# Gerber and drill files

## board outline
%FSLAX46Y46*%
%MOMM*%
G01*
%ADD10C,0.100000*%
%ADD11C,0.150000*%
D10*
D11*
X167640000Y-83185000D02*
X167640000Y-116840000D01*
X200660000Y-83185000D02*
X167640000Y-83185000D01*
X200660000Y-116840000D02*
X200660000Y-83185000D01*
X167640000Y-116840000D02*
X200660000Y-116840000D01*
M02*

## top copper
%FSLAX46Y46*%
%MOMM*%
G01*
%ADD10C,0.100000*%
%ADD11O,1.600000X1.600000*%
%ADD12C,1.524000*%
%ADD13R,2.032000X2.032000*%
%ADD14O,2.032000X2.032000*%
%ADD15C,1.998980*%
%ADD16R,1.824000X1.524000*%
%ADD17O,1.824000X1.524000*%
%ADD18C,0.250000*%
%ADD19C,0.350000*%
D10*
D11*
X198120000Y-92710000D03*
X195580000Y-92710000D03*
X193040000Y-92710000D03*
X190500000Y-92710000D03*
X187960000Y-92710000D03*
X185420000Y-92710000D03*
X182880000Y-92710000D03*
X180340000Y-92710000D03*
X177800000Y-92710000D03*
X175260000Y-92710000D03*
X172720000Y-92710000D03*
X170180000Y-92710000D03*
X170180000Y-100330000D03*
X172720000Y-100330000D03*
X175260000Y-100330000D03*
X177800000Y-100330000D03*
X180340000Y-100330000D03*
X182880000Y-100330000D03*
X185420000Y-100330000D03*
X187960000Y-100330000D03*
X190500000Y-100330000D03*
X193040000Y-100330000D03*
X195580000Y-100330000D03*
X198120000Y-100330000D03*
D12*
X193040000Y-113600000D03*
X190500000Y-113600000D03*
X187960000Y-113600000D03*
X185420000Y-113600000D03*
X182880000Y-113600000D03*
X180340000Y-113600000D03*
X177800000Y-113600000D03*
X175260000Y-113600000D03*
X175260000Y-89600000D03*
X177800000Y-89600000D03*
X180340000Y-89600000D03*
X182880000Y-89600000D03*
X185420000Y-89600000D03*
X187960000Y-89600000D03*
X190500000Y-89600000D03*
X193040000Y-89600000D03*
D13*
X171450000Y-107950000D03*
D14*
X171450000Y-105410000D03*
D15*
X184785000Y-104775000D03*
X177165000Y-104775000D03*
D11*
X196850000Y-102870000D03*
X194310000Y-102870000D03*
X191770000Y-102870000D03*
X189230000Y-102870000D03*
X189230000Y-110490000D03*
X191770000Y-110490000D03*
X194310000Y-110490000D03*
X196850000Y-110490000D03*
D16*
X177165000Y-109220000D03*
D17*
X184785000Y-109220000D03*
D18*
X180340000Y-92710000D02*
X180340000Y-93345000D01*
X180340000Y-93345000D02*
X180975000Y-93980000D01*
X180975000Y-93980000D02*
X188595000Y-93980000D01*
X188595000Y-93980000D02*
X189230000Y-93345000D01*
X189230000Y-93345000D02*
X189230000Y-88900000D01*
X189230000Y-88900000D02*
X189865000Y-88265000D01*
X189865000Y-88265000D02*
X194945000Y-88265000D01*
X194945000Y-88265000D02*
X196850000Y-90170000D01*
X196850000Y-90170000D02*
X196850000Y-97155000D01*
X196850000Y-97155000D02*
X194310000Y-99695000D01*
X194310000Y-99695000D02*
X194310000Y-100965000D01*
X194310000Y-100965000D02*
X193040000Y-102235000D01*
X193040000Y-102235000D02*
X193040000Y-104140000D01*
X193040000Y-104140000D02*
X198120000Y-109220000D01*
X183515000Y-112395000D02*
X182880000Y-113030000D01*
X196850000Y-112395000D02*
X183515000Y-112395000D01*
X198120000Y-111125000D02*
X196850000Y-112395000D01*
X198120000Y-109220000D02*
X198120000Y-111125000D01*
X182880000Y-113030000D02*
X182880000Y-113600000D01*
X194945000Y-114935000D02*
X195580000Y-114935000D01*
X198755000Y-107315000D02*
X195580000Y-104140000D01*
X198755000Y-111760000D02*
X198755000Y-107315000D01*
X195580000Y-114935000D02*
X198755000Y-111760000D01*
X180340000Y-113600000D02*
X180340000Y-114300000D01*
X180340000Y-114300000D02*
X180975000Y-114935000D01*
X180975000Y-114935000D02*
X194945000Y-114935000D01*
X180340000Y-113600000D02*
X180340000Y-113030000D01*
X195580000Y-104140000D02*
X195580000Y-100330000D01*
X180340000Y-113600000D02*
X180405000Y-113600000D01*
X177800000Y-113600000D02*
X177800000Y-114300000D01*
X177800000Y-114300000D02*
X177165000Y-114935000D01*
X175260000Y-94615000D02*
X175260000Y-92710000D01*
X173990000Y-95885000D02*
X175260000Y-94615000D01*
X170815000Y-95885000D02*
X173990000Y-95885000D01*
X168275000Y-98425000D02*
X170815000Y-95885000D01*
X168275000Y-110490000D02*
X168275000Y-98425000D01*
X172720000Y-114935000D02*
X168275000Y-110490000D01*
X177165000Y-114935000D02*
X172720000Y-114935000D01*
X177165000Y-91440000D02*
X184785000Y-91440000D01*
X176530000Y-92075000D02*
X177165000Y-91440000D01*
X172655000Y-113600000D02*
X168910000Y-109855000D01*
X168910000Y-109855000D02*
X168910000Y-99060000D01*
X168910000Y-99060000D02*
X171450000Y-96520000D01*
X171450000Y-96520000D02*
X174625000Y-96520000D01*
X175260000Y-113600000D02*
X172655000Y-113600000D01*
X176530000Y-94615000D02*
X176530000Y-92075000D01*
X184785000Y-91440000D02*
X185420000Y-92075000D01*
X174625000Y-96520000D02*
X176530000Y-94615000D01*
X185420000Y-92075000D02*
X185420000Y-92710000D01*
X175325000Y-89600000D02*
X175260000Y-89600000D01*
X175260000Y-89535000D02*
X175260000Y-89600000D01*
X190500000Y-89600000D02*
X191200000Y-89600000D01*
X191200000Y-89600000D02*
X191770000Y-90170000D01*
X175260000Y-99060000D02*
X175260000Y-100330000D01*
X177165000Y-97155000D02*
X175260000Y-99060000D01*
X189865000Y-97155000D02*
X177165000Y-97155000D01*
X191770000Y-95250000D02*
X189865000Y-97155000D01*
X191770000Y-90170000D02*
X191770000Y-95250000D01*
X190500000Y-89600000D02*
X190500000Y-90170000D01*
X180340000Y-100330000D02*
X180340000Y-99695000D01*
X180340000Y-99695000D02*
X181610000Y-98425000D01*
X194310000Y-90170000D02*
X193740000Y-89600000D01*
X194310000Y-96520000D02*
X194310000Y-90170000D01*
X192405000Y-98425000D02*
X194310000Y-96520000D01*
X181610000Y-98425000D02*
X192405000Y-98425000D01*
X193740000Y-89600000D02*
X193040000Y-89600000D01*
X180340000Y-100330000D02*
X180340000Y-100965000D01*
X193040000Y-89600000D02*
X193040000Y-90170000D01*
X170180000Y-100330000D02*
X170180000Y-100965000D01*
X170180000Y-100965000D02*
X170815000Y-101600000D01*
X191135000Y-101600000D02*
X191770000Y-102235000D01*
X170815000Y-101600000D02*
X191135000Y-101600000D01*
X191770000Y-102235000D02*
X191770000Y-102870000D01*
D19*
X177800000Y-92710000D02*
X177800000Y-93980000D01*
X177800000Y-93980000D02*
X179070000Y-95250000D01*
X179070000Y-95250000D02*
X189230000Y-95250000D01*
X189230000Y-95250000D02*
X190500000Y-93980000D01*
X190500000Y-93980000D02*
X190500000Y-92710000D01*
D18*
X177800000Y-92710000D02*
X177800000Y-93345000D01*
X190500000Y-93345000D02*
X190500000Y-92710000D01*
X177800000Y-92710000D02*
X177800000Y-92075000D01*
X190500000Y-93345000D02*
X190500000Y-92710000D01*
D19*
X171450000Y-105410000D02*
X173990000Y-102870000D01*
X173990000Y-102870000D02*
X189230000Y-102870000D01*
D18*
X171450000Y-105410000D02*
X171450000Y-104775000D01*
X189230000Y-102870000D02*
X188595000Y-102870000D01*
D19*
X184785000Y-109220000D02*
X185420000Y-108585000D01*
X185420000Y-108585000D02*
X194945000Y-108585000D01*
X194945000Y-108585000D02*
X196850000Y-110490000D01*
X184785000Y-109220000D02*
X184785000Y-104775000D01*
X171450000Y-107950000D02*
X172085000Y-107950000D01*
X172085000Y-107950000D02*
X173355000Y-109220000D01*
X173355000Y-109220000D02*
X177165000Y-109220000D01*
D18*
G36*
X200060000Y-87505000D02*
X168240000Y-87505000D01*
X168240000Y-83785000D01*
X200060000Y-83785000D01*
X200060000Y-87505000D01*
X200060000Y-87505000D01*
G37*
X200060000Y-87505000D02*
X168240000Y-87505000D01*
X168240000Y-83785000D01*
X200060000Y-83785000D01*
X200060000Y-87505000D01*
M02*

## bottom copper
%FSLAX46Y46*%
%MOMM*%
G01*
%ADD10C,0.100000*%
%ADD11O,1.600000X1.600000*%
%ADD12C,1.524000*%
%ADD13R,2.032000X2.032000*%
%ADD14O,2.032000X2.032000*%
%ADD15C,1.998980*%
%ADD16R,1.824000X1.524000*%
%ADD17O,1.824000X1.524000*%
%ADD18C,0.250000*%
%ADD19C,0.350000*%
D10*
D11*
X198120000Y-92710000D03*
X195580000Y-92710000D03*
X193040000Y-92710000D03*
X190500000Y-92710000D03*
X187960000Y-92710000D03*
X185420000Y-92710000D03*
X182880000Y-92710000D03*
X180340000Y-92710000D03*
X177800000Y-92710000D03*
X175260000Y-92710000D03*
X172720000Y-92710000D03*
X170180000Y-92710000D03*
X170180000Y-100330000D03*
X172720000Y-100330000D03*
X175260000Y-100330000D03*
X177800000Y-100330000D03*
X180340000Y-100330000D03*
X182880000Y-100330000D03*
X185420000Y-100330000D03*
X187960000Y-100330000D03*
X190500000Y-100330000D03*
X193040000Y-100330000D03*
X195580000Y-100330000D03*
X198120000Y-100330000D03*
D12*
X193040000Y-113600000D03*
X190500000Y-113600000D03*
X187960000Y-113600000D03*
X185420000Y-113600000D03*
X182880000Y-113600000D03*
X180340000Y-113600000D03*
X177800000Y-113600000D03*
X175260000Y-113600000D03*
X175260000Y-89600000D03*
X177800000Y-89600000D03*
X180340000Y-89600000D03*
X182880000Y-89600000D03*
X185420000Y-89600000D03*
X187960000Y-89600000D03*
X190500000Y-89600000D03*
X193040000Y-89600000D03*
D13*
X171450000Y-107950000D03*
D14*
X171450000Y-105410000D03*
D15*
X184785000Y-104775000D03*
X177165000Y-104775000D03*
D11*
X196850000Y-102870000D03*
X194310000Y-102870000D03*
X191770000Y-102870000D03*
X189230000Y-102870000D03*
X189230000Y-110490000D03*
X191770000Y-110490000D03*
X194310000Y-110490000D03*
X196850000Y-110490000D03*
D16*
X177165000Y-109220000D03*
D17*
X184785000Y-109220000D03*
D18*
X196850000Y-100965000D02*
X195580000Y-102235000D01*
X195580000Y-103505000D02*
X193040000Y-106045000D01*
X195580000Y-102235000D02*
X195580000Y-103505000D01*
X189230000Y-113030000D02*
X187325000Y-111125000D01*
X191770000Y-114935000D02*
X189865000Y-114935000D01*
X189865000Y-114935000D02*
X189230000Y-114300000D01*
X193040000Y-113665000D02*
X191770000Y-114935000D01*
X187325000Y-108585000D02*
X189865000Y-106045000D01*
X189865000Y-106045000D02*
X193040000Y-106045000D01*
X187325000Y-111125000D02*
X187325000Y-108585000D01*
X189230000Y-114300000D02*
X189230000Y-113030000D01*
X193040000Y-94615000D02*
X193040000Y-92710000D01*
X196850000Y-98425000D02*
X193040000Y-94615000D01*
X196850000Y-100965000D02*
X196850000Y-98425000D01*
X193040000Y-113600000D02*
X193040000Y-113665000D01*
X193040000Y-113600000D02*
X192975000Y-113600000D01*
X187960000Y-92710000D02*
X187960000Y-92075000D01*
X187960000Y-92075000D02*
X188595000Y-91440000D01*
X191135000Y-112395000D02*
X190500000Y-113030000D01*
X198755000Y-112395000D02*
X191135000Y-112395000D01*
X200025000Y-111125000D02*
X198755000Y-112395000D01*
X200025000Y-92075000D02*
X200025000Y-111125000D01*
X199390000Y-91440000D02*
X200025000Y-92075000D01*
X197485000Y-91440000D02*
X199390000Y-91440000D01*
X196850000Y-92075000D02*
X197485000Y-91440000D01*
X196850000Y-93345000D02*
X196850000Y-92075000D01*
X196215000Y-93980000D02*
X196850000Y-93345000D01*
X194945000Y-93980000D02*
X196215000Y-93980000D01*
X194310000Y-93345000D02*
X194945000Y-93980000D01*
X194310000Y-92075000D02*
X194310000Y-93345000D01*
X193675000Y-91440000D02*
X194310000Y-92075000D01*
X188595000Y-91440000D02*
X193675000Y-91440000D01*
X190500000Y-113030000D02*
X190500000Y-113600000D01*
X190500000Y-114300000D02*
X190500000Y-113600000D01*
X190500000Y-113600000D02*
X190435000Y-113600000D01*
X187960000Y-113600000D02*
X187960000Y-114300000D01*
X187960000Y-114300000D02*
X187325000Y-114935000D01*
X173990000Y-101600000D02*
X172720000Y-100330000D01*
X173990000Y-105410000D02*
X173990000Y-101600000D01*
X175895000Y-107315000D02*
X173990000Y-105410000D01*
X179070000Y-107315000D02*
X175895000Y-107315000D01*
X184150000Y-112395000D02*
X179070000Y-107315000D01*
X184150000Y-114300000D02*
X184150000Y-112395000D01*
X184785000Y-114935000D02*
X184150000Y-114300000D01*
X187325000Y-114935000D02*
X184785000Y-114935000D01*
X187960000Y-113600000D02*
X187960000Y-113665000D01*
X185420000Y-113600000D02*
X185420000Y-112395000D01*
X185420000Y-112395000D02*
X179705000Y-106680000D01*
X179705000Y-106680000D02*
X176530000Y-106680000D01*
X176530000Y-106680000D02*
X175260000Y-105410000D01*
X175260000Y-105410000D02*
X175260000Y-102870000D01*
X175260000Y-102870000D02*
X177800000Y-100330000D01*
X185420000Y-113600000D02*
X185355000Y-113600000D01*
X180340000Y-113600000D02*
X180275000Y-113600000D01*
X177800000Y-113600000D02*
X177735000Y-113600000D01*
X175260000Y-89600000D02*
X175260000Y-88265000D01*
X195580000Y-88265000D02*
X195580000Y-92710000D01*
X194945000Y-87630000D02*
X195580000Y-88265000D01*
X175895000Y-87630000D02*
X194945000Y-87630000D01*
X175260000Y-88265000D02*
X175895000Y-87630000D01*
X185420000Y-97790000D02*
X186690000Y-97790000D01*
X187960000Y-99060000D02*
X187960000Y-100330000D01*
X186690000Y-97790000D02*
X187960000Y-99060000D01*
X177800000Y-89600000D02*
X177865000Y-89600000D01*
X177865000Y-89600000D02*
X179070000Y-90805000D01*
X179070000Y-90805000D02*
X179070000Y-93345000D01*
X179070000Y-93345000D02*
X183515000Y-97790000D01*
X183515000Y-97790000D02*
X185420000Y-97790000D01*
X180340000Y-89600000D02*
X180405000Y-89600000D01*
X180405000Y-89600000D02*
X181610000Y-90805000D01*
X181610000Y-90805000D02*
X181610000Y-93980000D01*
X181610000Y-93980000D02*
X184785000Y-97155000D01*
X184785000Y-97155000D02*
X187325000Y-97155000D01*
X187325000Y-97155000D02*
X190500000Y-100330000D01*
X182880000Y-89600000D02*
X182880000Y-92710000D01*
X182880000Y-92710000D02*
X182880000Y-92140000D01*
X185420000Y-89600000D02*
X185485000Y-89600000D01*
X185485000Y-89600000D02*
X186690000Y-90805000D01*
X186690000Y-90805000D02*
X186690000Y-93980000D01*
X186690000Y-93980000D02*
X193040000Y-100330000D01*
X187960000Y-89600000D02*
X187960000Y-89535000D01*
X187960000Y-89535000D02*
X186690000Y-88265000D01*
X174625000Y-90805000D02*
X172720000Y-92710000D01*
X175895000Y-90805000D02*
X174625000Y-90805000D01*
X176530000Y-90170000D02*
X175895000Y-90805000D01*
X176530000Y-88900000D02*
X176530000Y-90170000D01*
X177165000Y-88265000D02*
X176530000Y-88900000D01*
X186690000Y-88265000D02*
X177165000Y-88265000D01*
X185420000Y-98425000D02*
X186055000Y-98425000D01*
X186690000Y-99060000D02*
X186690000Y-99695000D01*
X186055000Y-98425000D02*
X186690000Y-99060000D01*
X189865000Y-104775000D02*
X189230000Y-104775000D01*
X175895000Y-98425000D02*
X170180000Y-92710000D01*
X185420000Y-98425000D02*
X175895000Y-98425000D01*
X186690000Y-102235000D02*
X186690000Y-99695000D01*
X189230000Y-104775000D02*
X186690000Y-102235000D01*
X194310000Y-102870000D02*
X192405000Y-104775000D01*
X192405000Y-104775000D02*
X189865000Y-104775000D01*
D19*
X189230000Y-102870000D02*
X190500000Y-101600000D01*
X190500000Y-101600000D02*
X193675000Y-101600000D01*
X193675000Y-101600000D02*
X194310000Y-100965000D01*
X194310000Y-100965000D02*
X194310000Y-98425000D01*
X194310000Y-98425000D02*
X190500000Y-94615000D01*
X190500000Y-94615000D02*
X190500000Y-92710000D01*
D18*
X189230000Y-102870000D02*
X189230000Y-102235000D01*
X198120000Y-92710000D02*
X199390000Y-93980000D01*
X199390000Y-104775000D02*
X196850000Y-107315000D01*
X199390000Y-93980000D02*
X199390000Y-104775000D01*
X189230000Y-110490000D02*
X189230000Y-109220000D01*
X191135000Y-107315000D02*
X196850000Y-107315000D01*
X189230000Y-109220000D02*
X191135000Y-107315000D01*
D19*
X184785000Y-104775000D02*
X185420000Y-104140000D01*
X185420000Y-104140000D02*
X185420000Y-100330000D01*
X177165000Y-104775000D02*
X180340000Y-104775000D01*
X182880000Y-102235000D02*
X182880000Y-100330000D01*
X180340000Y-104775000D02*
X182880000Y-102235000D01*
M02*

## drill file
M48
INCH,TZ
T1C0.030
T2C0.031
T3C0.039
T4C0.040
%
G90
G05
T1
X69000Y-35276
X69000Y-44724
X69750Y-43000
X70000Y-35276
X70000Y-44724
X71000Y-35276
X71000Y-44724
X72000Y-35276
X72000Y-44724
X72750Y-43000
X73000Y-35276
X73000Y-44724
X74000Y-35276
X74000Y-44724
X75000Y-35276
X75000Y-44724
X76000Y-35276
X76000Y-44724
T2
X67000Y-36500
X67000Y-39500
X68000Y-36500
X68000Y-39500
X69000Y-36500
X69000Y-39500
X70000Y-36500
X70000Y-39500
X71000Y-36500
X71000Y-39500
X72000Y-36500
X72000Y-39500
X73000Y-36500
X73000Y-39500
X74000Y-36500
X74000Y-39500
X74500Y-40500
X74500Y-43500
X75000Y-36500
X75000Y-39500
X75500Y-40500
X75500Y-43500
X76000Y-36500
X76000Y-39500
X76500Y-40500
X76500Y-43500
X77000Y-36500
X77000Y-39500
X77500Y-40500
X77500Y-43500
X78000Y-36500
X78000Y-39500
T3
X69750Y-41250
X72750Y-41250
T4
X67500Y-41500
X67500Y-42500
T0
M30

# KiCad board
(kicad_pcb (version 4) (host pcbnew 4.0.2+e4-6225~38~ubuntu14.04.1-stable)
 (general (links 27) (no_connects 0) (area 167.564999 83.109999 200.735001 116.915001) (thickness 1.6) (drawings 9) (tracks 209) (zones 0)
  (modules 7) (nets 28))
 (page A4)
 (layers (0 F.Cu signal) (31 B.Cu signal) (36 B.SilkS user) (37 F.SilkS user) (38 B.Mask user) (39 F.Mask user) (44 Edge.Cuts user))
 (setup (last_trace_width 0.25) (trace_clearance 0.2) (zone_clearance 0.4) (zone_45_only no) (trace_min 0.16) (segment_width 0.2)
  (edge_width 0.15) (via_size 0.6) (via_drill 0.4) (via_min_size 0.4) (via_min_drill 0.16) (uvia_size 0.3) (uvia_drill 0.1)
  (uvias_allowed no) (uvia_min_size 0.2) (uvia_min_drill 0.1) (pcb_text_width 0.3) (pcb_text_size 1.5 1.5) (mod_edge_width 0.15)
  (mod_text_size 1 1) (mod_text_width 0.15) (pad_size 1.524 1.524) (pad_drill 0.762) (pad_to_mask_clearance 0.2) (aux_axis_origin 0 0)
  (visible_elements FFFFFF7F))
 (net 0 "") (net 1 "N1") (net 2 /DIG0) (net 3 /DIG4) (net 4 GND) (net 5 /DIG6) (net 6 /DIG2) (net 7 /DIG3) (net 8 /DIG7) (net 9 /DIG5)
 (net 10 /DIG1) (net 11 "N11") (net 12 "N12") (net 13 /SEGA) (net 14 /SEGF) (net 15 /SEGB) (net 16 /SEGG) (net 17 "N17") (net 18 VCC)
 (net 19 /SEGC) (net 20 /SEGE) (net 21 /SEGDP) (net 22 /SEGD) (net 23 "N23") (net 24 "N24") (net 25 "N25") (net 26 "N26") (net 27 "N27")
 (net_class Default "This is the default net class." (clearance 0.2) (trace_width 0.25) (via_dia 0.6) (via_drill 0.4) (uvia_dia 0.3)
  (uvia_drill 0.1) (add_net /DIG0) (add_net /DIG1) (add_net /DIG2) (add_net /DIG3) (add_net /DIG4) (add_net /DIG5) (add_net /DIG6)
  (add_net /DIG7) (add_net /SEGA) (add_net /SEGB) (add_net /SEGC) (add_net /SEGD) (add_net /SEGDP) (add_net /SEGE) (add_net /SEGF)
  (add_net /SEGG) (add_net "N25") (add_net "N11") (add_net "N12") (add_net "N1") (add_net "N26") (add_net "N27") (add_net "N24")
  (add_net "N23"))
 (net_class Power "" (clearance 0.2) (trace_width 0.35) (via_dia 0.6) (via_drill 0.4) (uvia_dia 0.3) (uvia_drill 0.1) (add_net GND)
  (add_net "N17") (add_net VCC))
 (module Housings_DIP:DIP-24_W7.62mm (layer F.Cu) (at 198.12 92.71 270)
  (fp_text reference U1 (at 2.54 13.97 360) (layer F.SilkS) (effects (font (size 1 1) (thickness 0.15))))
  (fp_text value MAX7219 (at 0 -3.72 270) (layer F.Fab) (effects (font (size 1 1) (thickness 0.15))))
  (pad 1 thru_hole oval (at 0 0 270) (size 1.6 1.6) (drill 0.8) (layers *.Cu *.Mask F.SilkS) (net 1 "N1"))
  (pad 2 thru_hole oval (at 0 2.54 270) (size 1.6 1.6) (drill 0.8) (layers *.Cu *.Mask F.SilkS) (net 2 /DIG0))
  (pad 3 thru_hole oval (at 0 5.08 270) (size 1.6 1.6) (drill 0.8) (layers *.Cu *.Mask F.SilkS) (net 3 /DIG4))
  (pad 4 thru_hole oval (at 0 7.62 270) (size 1.6 1.6) (drill 0.8) (layers *.Cu *.Mask F.SilkS) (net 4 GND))
  (pad 5 thru_hole oval (at 0 10.16 270) (size 1.6 1.6) (drill 0.8) (layers *.Cu *.Mask F.SilkS) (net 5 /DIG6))
  (pad 6 thru_hole oval (at 0 12.7 270) (size 1.6 1.6) (drill 0.8) (layers *.Cu *.Mask F.SilkS) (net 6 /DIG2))
  (pad 7 thru_hole oval (at 0 15.24 270) (size 1.6 1.6) (drill 0.8) (layers *.Cu *.Mask F.SilkS) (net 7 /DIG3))
  (pad 8 thru_hole oval (at 0 17.78 270) (size 1.6 1.6) (drill 0.8) (layers *.Cu *.Mask F.SilkS) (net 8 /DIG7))
  (pad 9 thru_hole oval (at 0 20.32 270) (size 1.6 1.6) (drill 0.8) (layers *.Cu *.Mask F.SilkS) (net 4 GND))
  (pad 10 thru_hole oval (at 0 22.86 270) (size 1.6 1.6) (drill 0.8) (layers *.Cu *.Mask F.SilkS) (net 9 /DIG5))
  (pad 11 thru_hole oval (at 0 25.4 270) (size 1.6 1.6) (drill 0.8) (layers *.Cu *.Mask F.SilkS) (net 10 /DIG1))
  (pad 12 thru_hole oval (at 0 27.94 270) (size 1.6 1.6) (drill 0.8) (layers *.Cu *.Mask F.SilkS) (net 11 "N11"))
  (pad 13 thru_hole oval (at 7.62 27.94 270) (size 1.6 1.6) (drill 0.8) (layers *.Cu *.Mask F.SilkS) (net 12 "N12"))
  (pad 14 thru_hole oval (at 7.62 25.4 270) (size 1.6 1.6) (drill 0.8) (layers *.Cu *.Mask F.SilkS) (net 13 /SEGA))
  (pad 15 thru_hole oval (at 7.62 22.86 270) (size 1.6 1.6) (drill 0.8) (layers *.Cu *.Mask F.SilkS) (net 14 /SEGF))
  (pad 16 thru_hole oval (at 7.62 20.32 270) (size 1.6 1.6) (drill 0.8) (layers *.Cu *.Mask F.SilkS) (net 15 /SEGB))
  (pad 17 thru_hole oval (at 7.62 17.78 270) (size 1.6 1.6) (drill 0.8) (layers *.Cu *.Mask F.SilkS) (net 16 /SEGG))
  (pad 18 thru_hole oval (at 7.62 15.24 270) (size 1.6 1.6) (drill 0.8) (layers *.Cu *.Mask F.SilkS) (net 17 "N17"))
  (pad 19 thru_hole oval (at 7.62 12.7 270) (size 1.6 1.6) (drill 0.8) (layers *.Cu *.Mask F.SilkS) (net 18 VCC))
  (pad 20 thru_hole oval (at 7.62 10.16 270) (size 1.6 1.6) (drill 0.8) (layers *.Cu *.Mask F.SilkS) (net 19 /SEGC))
  (pad 21 thru_hole oval (at 7.62 7.62 270) (size 1.6 1.6) (drill 0.8) (layers *.Cu *.Mask F.SilkS) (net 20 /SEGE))
  (pad 22 thru_hole oval (at 7.62 5.08 270) (size 1.6 1.6) (drill 0.8) (layers *.Cu *.Mask F.SilkS) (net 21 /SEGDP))
  (pad 23 thru_hole oval (at 7.62 2.54 270) (size 1.6 1.6) (drill 0.8) (layers *.Cu *.Mask F.SilkS) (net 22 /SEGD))
  (pad 24 thru_hole oval (at 7.62 0 270) (size 1.6 1.6) (drill 0.8) (layers *.Cu *.Mask F.SilkS) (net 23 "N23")))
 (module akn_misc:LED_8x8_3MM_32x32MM (layer B.Cu) (at 184.15 101.6 90)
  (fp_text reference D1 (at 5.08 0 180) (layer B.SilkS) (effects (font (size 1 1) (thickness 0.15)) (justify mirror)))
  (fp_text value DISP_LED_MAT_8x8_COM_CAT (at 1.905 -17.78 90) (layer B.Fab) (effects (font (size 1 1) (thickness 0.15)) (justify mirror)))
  (pad 1 thru_hole circle (at -12 8.89 90) (size 1.524 1.524) (drill 0.762) (layers *.Cu *.Mask B.SilkS) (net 3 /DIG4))
  (pad 2 thru_hole circle (at -12 6.35 90) (size 1.524 1.524) (drill 0.762) (layers *.Cu *.Mask B.SilkS) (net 5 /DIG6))
  (pad 3 thru_hole circle (at -12 3.81 90) (size 1.524 1.524) (drill 0.762) (layers *.Cu *.Mask B.SilkS) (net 13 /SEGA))
  (pad 4 thru_hole circle (at -12 1.27 90) (size 1.524 1.524) (drill 0.762) (layers *.Cu *.Mask B.SilkS) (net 15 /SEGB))
  (pad 5 thru_hole circle (at -12 -1.27 90) (size 1.524 1.524) (drill 0.762) (layers *.Cu *.Mask B.SilkS) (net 8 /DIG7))
  (pad 6 thru_hole circle (at -12 -3.81 90) (size 1.524 1.524) (drill 0.762) (layers *.Cu *.Mask B.SilkS) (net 22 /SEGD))
  (pad 7 thru_hole circle (at -12 -6.35 90) (size 1.524 1.524) (drill 0.762) (layers *.Cu *.Mask B.SilkS) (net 9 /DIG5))
  (pad 8 thru_hole circle (at -12 -8.89 90) (size 1.524 1.524) (drill 0.762) (layers *.Cu *.Mask B.SilkS) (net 6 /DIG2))
  (pad 9 thru_hole circle (at 12 -8.89 90) (size 1.524 1.524) (drill 0.762) (layers *.Cu *.Mask B.SilkS) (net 2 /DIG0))
  (pad 10 thru_hole circle (at 12 -6.35 90) (size 1.524 1.524) (drill 0.762) (layers *.Cu *.Mask B.SilkS) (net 19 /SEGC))
  (pad 11 thru_hole circle (at 12 -3.81 90) (size 1.524 1.524) (drill 0.762) (layers *.Cu *.Mask B.SilkS) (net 20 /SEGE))
  (pad 12 thru_hole circle (at 12 -1.27 90) (size 1.524 1.524) (drill 0.762) (layers *.Cu *.Mask B.SilkS) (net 7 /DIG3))
  (pad 13 thru_hole circle (at 12 1.27 90) (size 1.524 1.524) (drill 0.762) (layers *.Cu *.Mask B.SilkS) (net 21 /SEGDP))
  (pad 14 thru_hole circle (at 12 3.81 90) (size 1.524 1.524) (drill 0.762) (layers *.Cu *.Mask B.SilkS) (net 10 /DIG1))
  (pad 15 thru_hole circle (at 12 6.35 90) (size 1.524 1.524) (drill 0.762) (layers *.Cu *.Mask B.SilkS) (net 14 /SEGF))
  (pad 16 thru_hole circle (at 12 8.89 90) (size 1.524 1.524) (drill 0.762) (layers *.Cu *.Mask B.SilkS) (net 16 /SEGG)))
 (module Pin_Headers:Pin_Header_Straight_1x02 (layer F.Cu) (at 171.45 107.95 180)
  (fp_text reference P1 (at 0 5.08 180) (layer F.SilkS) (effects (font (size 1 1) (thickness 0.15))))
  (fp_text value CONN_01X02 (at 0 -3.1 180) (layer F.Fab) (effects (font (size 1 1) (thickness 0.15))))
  (pad 1 thru_hole rect (at 0 0 180) (size 2.032 2.032) (drill 1.016) (layers *.Cu *.Mask F.SilkS) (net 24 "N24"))
  (pad 2 thru_hole oval (at 0 2.54 180) (size 2.032 2.032) (drill 1.016) (layers *.Cu *.Mask F.SilkS) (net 4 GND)))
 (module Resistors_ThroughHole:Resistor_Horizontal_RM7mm (layer F.Cu) (at 184.785 104.775 180)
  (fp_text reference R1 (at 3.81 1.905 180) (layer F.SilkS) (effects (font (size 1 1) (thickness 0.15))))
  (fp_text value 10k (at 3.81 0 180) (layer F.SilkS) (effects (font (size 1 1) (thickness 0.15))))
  (pad 1 thru_hole circle (at 0 0 180) (size 1.99898 1.99898) (drill 1.00076) (layers *.Cu *.SilkS *.Mask) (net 18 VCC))
  (pad 2 thru_hole circle (at 7.62 0 180) (size 1.99898 1.99898) (drill 1.00076) (layers *.Cu *.SilkS *.Mask) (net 17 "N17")))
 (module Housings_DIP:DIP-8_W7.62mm (layer F.Cu) (at 196.85 102.87 270)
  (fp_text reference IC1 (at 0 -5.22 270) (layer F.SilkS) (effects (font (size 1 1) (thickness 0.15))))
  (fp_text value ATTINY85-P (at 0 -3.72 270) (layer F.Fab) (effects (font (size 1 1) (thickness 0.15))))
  (pad 1 thru_hole oval (at 0 0 270) (size 1.6 1.6) (drill 0.8) (layers *.Cu *.Mask F.SilkS) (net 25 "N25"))
  (pad 2 thru_hole oval (at 0 2.54 270) (size 1.6 1.6) (drill 0.8) (layers *.Cu *.Mask F.SilkS) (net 11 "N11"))
  (pad 3 thru_hole oval (at 0 5.08 270) (size 1.6 1.6) (drill 0.8) (layers *.Cu *.Mask F.SilkS) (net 12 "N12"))
  (pad 4 thru_hole oval (at 0 7.62 270) (size 1.6 1.6) (drill 0.8) (layers *.Cu *.Mask F.SilkS) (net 4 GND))
  (pad 5 thru_hole oval (at 7.62 7.62 270) (size 1.6 1.6) (drill 0.8) (layers *.Cu *.Mask F.SilkS) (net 1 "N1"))
  (pad 6 thru_hole oval (at 7.62 5.08 270) (size 1.6 1.6) (drill 0.8) (layers *.Cu *.Mask F.SilkS) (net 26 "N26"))
  (pad 7 thru_hole oval (at 7.62 2.54 270) (size 1.6 1.6) (drill 0.8) (layers *.Cu *.Mask F.SilkS) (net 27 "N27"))
  (pad 8 thru_hole oval (at 7.62 0 270) (size 1.6 1.6) (drill 0.8) (layers *.Cu *.Mask F.SilkS) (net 18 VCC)))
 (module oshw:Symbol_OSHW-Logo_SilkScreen (layer B.Cu) (at 187.96 86.36 180)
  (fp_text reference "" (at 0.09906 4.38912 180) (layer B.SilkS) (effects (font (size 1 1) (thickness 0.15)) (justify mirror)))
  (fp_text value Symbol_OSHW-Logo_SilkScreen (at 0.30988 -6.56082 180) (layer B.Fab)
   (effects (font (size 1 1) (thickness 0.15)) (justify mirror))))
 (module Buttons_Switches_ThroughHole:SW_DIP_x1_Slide (layer F.Cu) (at 177.165 109.22 270)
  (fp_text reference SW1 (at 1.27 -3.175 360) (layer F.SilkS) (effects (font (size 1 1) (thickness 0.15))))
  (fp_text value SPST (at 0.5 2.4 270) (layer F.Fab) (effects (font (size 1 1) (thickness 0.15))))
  (pad 1 thru_hole rect (at 0 0 270) (size 1.524 1.824) (drill 0.762) (layers *.Cu *.Mask F.SilkS) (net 24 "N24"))
  (pad 2 thru_hole oval (at 0 -7.62 270) (size 1.524 1.824) (drill 0.762) (layers *.Cu *.Mask F.SilkS) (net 18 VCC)))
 (gr_line (start 167.64 83.185) (end 167.64 116.84) (angle 90) (layer Edge.Cuts) (width 0.15))
 (gr_line (start 200.66 83.185) (end 167.64 83.185) (angle 90) (layer Edge.Cuts) (width 0.15))
 (gr_line (start 200.66 116.84) (end 200.66 83.185) (angle 90) (layer Edge.Cuts) (width 0.15))
 (gr_line (start 167.64 116.84) (end 200.66 116.84) (angle 90) (layer Edge.Cuts) (width 0.15))
 (segment (start 196.85 100.965) (end 195.58 102.235) (width 0.25) (layer B.Cu) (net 3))
 (segment (start 195.58 103.505) (end 193.04 106.045) (width 0.25) (layer B.Cu) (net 3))
 (segment (start 195.58 102.235) (end 195.58 103.505) (width 0.25) (layer B.Cu) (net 3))
 (segment (start 189.23 113.03) (end 187.325 111.125) (width 0.25) (layer B.Cu) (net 3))
 (segment (start 191.77 114.935) (end 189.865 114.935) (width 0.25) (layer B.Cu) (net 3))
 (segment (start 189.865 114.935) (end 189.23 114.3) (width 0.25) (layer B.Cu) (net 3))
 (segment (start 193.04 113.665) (end 191.77 114.935) (width 0.25) (layer B.Cu) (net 3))
 (segment (start 187.325 108.585) (end 189.865 106.045) (width 0.25) (layer B.Cu) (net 3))
 (segment (start 189.865 106.045) (end 193.04 106.045) (width 0.25) (layer B.Cu) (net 3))
 (segment (start 187.325 111.125) (end 187.325 108.585) (width 0.25) (layer B.Cu) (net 3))
 (segment (start 189.23 114.3) (end 189.23 113.03) (width 0.25) (layer B.Cu) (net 3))
 (segment (start 193.04 94.615) (end 193.04 92.71) (width 0.25) (layer B.Cu) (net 3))
 (segment (start 196.85 98.425) (end 193.04 94.615) (width 0.25) (layer B.Cu) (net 3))
 (segment (start 196.85 100.965) (end 196.85 98.425) (width 0.25) (layer B.Cu) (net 3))
 (segment (start 193.04 113.6) (end 193.04 113.665) (width 0.25) (layer B.Cu) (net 3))
 (segment (start 193.04 113.6) (end 192.975 113.6) (width 0.25) (layer B.Cu) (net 3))
 (segment (start 187.96 92.71) (end 187.96 92.075) (width 0.25) (layer B.Cu) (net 5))
 (segment (start 187.96 92.075) (end 188.595 91.44) (width 0.25) (layer B.Cu) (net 5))
 (segment (start 191.135 112.395) (end 190.5 113.03) (width 0.25) (layer B.Cu) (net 5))
 (segment (start 198.755 112.395) (end 191.135 112.395) (width 0.25) (layer B.Cu) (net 5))
 (segment (start 200.025 111.125) (end 198.755 112.395) (width 0.25) (layer B.Cu) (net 5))
 (segment (start 200.025 92.075) (end 200.025 111.125) (width 0.25) (layer B.Cu) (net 5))
 (segment (start 199.39 91.44) (end 200.025 92.075) (width 0.25) (layer B.Cu) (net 5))
 (segment (start 197.485 91.44) (end 199.39 91.44) (width 0.25) (layer B.Cu) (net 5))
 (segment (start 196.85 92.075) (end 197.485 91.44) (width 0.25) (layer B.Cu) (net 5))
 (segment (start 196.85 93.345) (end 196.85 92.075) (width 0.25) (layer B.Cu) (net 5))
 (segment (start 196.215 93.98) (end 196.85 93.345) (width 0.25) (layer B.Cu) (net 5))
 (segment (start 194.945 93.98) (end 196.215 93.98) (width 0.25) (layer B.Cu) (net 5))
 (segment (start 194.31 93.345) (end 194.945 93.98) (width 0.25) (layer B.Cu) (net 5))
 (segment (start 194.31 92.075) (end 194.31 93.345) (width 0.25) (layer B.Cu) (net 5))
 (segment (start 193.675 91.44) (end 194.31 92.075) (width 0.25) (layer B.Cu) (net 5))
 (segment (start 188.595 91.44) (end 193.675 91.44) (width 0.25) (layer B.Cu) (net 5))
 (segment (start 190.5 113.03) (end 190.5 113.6) (width 0.25) (layer B.Cu) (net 5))
 (segment (start 190.5 114.3) (end 190.5 113.6) (width 0.25) (layer B.Cu) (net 5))
 (segment (start 190.5 113.6) (end 190.435 113.6) (width 0.25) (layer B.Cu) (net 5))
 (segment (start 187.96 113.6) (end 187.96 114.3) (width 0.25) (layer B.Cu) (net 13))
 (segment (start 187.96 114.3) (end 187.325 114.935) (width 0.25) (layer B.Cu) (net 13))
 (segment (start 173.99 101.6) (end 172.72 100.33) (width 0.25) (layer B.Cu) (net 13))
 (segment (start 173.99 105.41) (end 173.99 101.6) (width 0.25) (layer B.Cu) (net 13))
 (segment (start 175.895 107.315) (end 173.99 105.41) (width 0.25) (layer B.Cu) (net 13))
 (segment (start 179.07 107.315) (end 175.895 107.315) (width 0.25) (layer B.Cu) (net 13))
 (segment (start 184.15 112.395) (end 179.07 107.315) (width 0.25) (layer B.Cu) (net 13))
 (segment (start 184.15 114.3) (end 184.15 112.395) (width 0.25) (layer B.Cu) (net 13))
 (segment (start 184.785 114.935) (end 184.15 114.3) (width 0.25) (layer B.Cu) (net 13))
 (segment (start 187.325 114.935) (end 184.785 114.935) (width 0.25) (layer B.Cu) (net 13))
 (segment (start 187.96 113.6) (end 187.96 113.665) (width 0.25) (layer B.Cu) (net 13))
 (segment (start 185.42 113.6) (end 185.42 112.395) (width 0.25) (layer B.Cu) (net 15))
 (segment (start 185.42 112.395) (end 179.705 106.68) (width 0.25) (layer B.Cu) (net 15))
 (segment (start 179.705 106.68) (end 176.53 106.68) (width 0.25) (layer B.Cu) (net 15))
 (segment (start 176.53 106.68) (end 175.26 105.41) (width 0.25) (layer B.Cu) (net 15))
 (segment (start 175.26 105.41) (end 175.26 102.87) (width 0.25) (layer B.Cu) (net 15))
 (segment (start 175.26 102.87) (end 177.8 100.33) (width 0.25) (layer B.Cu) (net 15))
 (segment (start 185.42 113.6) (end 185.355 113.6) (width 0.25) (layer B.Cu) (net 15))
 (segment (start 180.34 92.71) (end 180.34 93.345) (width 0.25) (layer F.Cu) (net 8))
 (segment (start 180.34 93.345) (end 180.975 93.98) (width 0.25) (layer F.Cu) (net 8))
 (segment (start 180.975 93.98) (end 188.595 93.98) (width 0.25) (layer F.Cu) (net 8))
 (segment (start 188.595 93.98) (end 189.23 93.345) (width 0.25) (layer F.Cu) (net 8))
 (segment (start 189.23 93.345) (end 189.23 88.9) (width 0.25) (layer F.Cu) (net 8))
 (segment (start 189.23 88.9) (end 189.865 88.265) (width 0.25) (layer F.Cu) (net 8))
 (segment (start 189.865 88.265) (end 194.945 88.265) (width 0.25) (layer F.Cu) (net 8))
 (segment (start 194.945 88.265) (end 196.85 90.17) (width 0.25) (layer F.Cu) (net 8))
 (segment (start 196.85 90.17) (end 196.85 97.155) (width 0.25) (layer F.Cu) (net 8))
 (segment (start 196.85 97.155) (end 194.31 99.695) (width 0.25) (layer F.Cu) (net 8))
 (segment (start 194.31 99.695) (end 194.31 100.965) (width 0.25) (layer F.Cu) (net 8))
 (segment (start 194.31 100.965) (end 193.04 102.235) (width 0.25) (layer F.Cu) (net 8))
 (segment (start 193.04 102.235) (end 193.04 104.14) (width 0.25) (layer F.Cu) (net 8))
 (segment (start 193.04 104.14) (end 198.12 109.22) (width 0.25) (layer F.Cu) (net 8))
 (segment (start 183.515 112.395) (end 182.88 113.03) (width 0.25) (layer F.Cu) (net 8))
 (segment (start 196.85 112.395) (end 183.515 112.395) (width 0.25) (layer F.Cu) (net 8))
 (segment (start 198.12 111.125) (end 196.85 112.395) (width 0.25) (layer F.Cu) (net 8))
 (segment (start 198.12 109.22) (end 198.12 111.125) (width 0.25) (layer F.Cu) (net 8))
 (segment (start 182.88 113.03) (end 182.88 113.6) (width 0.25) (layer F.Cu) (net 8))
 (segment (start 180.34 113.6) (end 180.275 113.6) (width 0.25) (layer B.Cu) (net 22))
 (segment (start 194.945 114.935) (end 195.58 114.935) (width 0.25) (layer F.Cu) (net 22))
 (segment (start 198.755 107.315) (end 195.58 104.14) (width 0.25) (layer F.Cu) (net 22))
 (segment (start 198.755 111.76) (end 198.755 107.315) (width 0.25) (layer F.Cu) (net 22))
 (segment (start 195.58 114.935) (end 198.755 111.76) (width 0.25) (layer F.Cu) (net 22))
 (segment (start 180.34 113.6) (end 180.34 114.3) (width 0.25) (layer F.Cu) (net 22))
 (segment (start 180.34 114.3) (end 180.975 114.935) (width 0.25) (layer F.Cu) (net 22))
 (segment (start 180.975 114.935) (end 194.945 114.935) (width 0.25) (layer F.Cu) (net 22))
 (segment (start 180.34 113.6) (end 180.34 113.03) (width 0.25) (layer F.Cu) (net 22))
 (segment (start 195.58 104.14) (end 195.58 100.33) (width 0.25) (layer F.Cu) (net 22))
 (segment (start 180.34 113.6) (end 180.405 113.6) (width 0.25) (layer F.Cu) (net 22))
 (segment (start 177.8 113.6) (end 177.735 113.6) (width 0.25) (layer B.Cu) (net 9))
 (segment (start 177.8 113.6) (end 177.8 114.3) (width 0.25) (layer F.Cu) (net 9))
 (segment (start 177.8 114.3) (end 177.165 114.935) (width 0.25) (layer F.Cu) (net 9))
 (segment (start 175.26 94.615) (end 175.26 92.71) (width 0.25) (layer F.Cu) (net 9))
 (segment (start 173.99 95.885) (end 175.26 94.615) (width 0.25) (layer F.Cu) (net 9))
 (segment (start 170.815 95.885) (end 173.99 95.885) (width 0.25) (layer F.Cu) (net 9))
 (segment (start 168.275 98.425) (end 170.815 95.885) (width 0.25) (layer F.Cu) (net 9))
 (segment (start 168.275 110.49) (end 168.275 98.425) (width 0.25) (layer F.Cu) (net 9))
 (segment (start 172.72 114.935) (end 168.275 110.49) (width 0.25) (layer F.Cu) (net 9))
 (segment (start 177.165 114.935) (end 172.72 114.935) (width 0.25) (layer F.Cu) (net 9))
 (segment (start 177.165 91.44) (end 184.785 91.44) (width 0.25) (layer F.Cu) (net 6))
 (segment (start 176.53 92.075) (end 177.165 91.44) (width 0.25) (layer F.Cu) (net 6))
 (segment (start 172.655 113.6) (end 168.91 109.855) (width 0.25) (layer F.Cu) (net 6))
 (segment (start 168.91 109.855) (end 168.91 99.06) (width 0.25) (layer F.Cu) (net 6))
 (segment (start 168.91 99.06) (end 171.45 96.52) (width 0.25) (layer F.Cu) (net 6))
 (segment (start 171.45 96.52) (end 174.625 96.52) (width 0.25) (layer F.Cu) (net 6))
 (segment (start 175.26 113.6) (end 172.655 113.6) (width 0.25) (layer F.Cu) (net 6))
 (segment (start 176.53 94.615) (end 176.53 92.075) (width 0.25) (layer F.Cu) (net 6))
 (segment (start 184.785 91.44) (end 185.42 92.075) (width 0.25) (layer F.Cu) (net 6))
 (segment (start 174.625 96.52) (end 176.53 94.615) (width 0.25) (layer F.Cu) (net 6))
 (segment (start 185.42 92.075) (end 185.42 92.71) (width 0.25) (layer F.Cu) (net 6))
 (segment (start 175.325 89.6) (end 175.26 89.6) (width 0.25) (layer F.Cu) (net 2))
 (segment (start 175.26 89.535) (end 175.26 89.6) (width 0.25) (layer F.Cu) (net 2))
 (segment (start 175.26 89.6) (end 175.26 88.265) (width 0.25) (layer B.Cu) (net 2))
 (segment (start 195.58 88.265) (end 195.58 92.71) (width 0.25) (layer B.Cu) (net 2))
 (segment (start 194.945 87.63) (end 195.58 88.265) (width 0.25) (layer B.Cu) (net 2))
 (segment (start 175.895 87.63) (end 194.945 87.63) (width 0.25) (layer B.Cu) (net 2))
 (segment (start 175.26 88.265) (end 175.895 87.63) (width 0.25) (layer B.Cu) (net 2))
 (segment (start 185.42 97.79) (end 186.69 97.79) (width 0.25) (layer B.Cu) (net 19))
 (segment (start 187.96 99.06) (end 187.96 100.33) (width 0.25) (layer B.Cu) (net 19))
 (segment (start 186.69 97.79) (end 187.96 99.06) (width 0.25) (layer B.Cu) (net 19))
 (segment (start 177.8 89.6) (end 177.865 89.6) (width 0.25) (layer B.Cu) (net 19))
 (segment (start 177.865 89.6) (end 179.07 90.805) (width 0.25) (layer B.Cu) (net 19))
 (segment (start 179.07 90.805) (end 179.07 93.345) (width 0.25) (layer B.Cu) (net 19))
 (segment (start 179.07 93.345) (end 183.515 97.79) (width 0.25) (layer B.Cu) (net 19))
 (segment (start 183.515 97.79) (end 185.42 97.79) (width 0.25) (layer B.Cu) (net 19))
 (segment (start 180.34 89.6) (end 180.405 89.6) (width 0.25) (layer B.Cu) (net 20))
 (segment (start 180.405 89.6) (end 181.61 90.805) (width 0.25) (layer B.Cu) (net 20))
 (segment (start 181.61 90.805) (end 181.61 93.98) (width 0.25) (layer B.Cu) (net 20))
 (segment (start 181.61 93.98) (end 184.785 97.155) (width 0.25) (layer B.Cu) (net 20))
 (segment (start 184.785 97.155) (end 187.325 97.155) (width 0.25) (layer B.Cu) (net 20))
 (segment (start 187.325 97.155) (end 190.5 100.33) (width 0.25) (layer B.Cu) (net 20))
 (segment (start 182.88 89.6) (end 182.88 92.71) (width 0.25) (layer B.Cu) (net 7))
 (segment (start 182.88 92.71) (end 182.88 92.14) (width 0.25) (layer B.Cu) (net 7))
 (segment (start 185.42 89.6) (end 185.485 89.6) (width 0.25) (layer B.Cu) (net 21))
 (segment (start 185.485 89.6) (end 186.69 90.805) (width 0.25) (layer B.Cu) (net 21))
 (segment (start 186.69 90.805) (end 186.69 93.98) (width 0.25) (layer B.Cu) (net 21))
 (segment (start 186.69 93.98) (end 193.04 100.33) (width 0.25) (layer B.Cu) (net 21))
 (segment (start 187.96 89.6) (end 187.96 89.535) (width 0.25) (layer B.Cu) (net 10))
 (segment (start 187.96 89.535) (end 186.69 88.265) (width 0.25) (layer B.Cu) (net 10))
 (segment (start 174.625 90.805) (end 172.72 92.71) (width 0.25) (layer B.Cu) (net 10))
 (segment (start 175.895 90.805) (end 174.625 90.805) (width 0.25) (layer B.Cu) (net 10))
 (segment (start 176.53 90.17) (end 175.895 90.805) (width 0.25) (layer B.Cu) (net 10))
 (segment (start 176.53 88.9) (end 176.53 90.17) (width 0.25) (layer B.Cu) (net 10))
 (segment (start 177.165 88.265) (end 176.53 88.9) (width 0.25) (layer B.Cu) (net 10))
 (segment (start 186.69 88.265) (end 177.165 88.265) (width 0.25) (layer B.Cu) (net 10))
 (segment (start 190.5 89.6) (end 191.2 89.6) (width 0.25) (layer F.Cu) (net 14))
 (segment (start 191.2 89.6) (end 191.77 90.17) (width 0.25) (layer F.Cu) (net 14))
 (segment (start 175.26 99.06) (end 175.26 100.33) (width 0.25) (layer F.Cu) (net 14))
 (segment (start 177.165 97.155) (end 175.26 99.06) (width 0.25) (layer F.Cu) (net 14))
 (segment (start 189.865 97.155) (end 177.165 97.155) (width 0.25) (layer F.Cu) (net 14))
 (segment (start 191.77 95.25) (end 189.865 97.155) (width 0.25) (layer F.Cu) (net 14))
 (segment (start 191.77 90.17) (end 191.77 95.25) (width 0.25) (layer F.Cu) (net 14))
 (segment (start 190.5 89.6) (end 190.5 90.17) (width 0.25) (layer F.Cu) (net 14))
 (segment (start 180.34 100.33) (end 180.34 99.695) (width 0.25) (layer F.Cu) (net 16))
 (segment (start 180.34 99.695) (end 181.61 98.425) (width 0.25) (layer F.Cu) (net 16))
 (segment (start 194.31 90.17) (end 193.74 89.6) (width 0.25) (layer F.Cu) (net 16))
 (segment (start 194.31 96.52) (end 194.31 90.17) (width 0.25) (layer F.Cu) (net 16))
 (segment (start 192.405 98.425) (end 194.31 96.52) (width 0.25) (layer F.Cu) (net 16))
 (segment (start 181.61 98.425) (end 192.405 98.425) (width 0.25) (layer F.Cu) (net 16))
 (segment (start 193.74 89.6) (end 193.04 89.6) (width 0.25) (layer F.Cu) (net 16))
 (segment (start 180.34 100.33) (end 180.34 100.965) (width 0.25) (layer F.Cu) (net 16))
 (segment (start 193.04 89.6) (end 193.04 90.17) (width 0.25) (layer F.Cu) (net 16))
 (segment (start 185.42 98.425) (end 186.055 98.425) (width 0.25) (layer B.Cu) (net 11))
 (segment (start 186.69 99.06) (end 186.69 99.695) (width 0.25) (layer B.Cu) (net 11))
 (segment (start 186.055 98.425) (end 186.69 99.06) (width 0.25) (layer B.Cu) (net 11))
 (segment (start 189.865 104.775) (end 189.23 104.775) (width 0.25) (layer B.Cu) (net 11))
 (segment (start 175.895 98.425) (end 170.18 92.71) (width 0.25) (layer B.Cu) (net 11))
 (segment (start 185.42 98.425) (end 175.895 98.425) (width 0.25) (layer B.Cu) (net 11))
 (segment (start 186.69 102.235) (end 186.69 99.695) (width 0.25) (layer B.Cu) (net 11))
 (segment (start 189.23 104.775) (end 186.69 102.235) (width 0.25) (layer B.Cu) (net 11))
 (segment (start 194.31 102.87) (end 192.405 104.775) (width 0.25) (layer B.Cu) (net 11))
 (segment (start 192.405 104.775) (end 189.865 104.775) (width 0.25) (layer B.Cu) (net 11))
 (segment (start 170.18 100.33) (end 170.18 100.965) (width 0.25) (layer F.Cu) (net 12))
 (segment (start 170.18 100.965) (end 170.815 101.6) (width 0.25) (layer F.Cu) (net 12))
 (segment (start 191.135 101.6) (end 191.77 102.235) (width 0.25) (layer F.Cu) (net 12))
 (segment (start 170.815 101.6) (end 191.135 101.6) (width 0.25) (layer F.Cu) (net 12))
 (segment (start 191.77 102.235) (end 191.77 102.87) (width 0.25) (layer F.Cu) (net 12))
 (segment (start 177.8 92.71) (end 177.8 93.98) (width 0.35) (layer F.Cu) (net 4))
 (segment (start 177.8 93.98) (end 179.07 95.25) (width 0.35) (layer F.Cu) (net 4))
 (segment (start 179.07 95.25) (end 189.23 95.25) (width 0.35) (layer F.Cu) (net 4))
 (segment (start 189.23 95.25) (end 190.5 93.98) (width 0.35) (layer F.Cu) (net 4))
 (segment (start 190.5 93.98) (end 190.5 92.71) (width 0.35) (layer F.Cu) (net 4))
 (segment (start 177.8 92.71) (end 177.8 93.345) (width 0.25) (layer F.Cu) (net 4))
 (segment (start 190.5 93.345) (end 190.5 92.71) (width 0.25) (layer F.Cu) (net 4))
 (segment (start 177.8 92.71) (end 177.8 92.075) (width 0.25) (layer F.Cu) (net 4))
 (segment (start 190.5 93.345) (end 190.5 92.71) (width 0.25) (layer F.Cu) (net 4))
 (segment (start 171.45 105.41) (end 173.99 102.87) (width 0.35) (layer F.Cu) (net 4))
 (segment (start 173.99 102.87) (end 189.23 102.87) (width 0.35) (layer F.Cu) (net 4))
 (segment (start 189.23 102.87) (end 190.5 101.6) (width 0.35) (layer B.Cu) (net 4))
 (segment (start 190.5 101.6) (end 193.675 101.6) (width 0.35) (layer B.Cu) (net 4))
 (segment (start 193.675 101.6) (end 194.31 100.965) (width 0.35) (layer B.Cu) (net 4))
 (segment (start 194.31 100.965) (end 194.31 98.425) (width 0.35) (layer B.Cu) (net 4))
 (segment (start 194.31 98.425) (end 190.5 94.615) (width 0.35) (layer B.Cu) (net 4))
 (segment (start 190.5 94.615) (end 190.5 92.71) (width 0.35) (layer B.Cu) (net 4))
 (segment (start 189.23 102.87) (end 189.23 102.235) (width 0.25) (layer B.Cu) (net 4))
 (segment (start 171.45 105.41) (end 171.45 104.775) (width 0.25) (layer F.Cu) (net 4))
 (segment (start 189.23 102.87) (end 188.595 102.87) (width 0.25) (layer F.Cu) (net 4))
 (segment (start 198.12 92.71) (end 199.39 93.98) (width 0.25) (layer B.Cu) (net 1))
 (segment (start 199.39 104.775) (end 196.85 107.315) (width 0.25) (layer B.Cu) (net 1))
 (segment (start 199.39 93.98) (end 199.39 104.775) (width 0.25) (layer B.Cu) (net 1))
 (segment (start 189.23 110.49) (end 189.23 109.22) (width 0.25) (layer B.Cu) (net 1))
 (segment (start 191.135 107.315) (end 196.85 107.315) (width 0.25) (layer B.Cu) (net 1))
 (segment (start 189.23 109.22) (end 191.135 107.315) (width 0.25) (layer B.Cu) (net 1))
 (segment (start 184.785 109.22) (end 185.42 108.585) (width 0.35) (layer F.Cu) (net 18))
 (segment (start 185.42 108.585) (end 194.945 108.585) (width 0.35) (layer F.Cu) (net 18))
 (segment (start 194.945 108.585) (end 196.85 110.49) (width 0.35) (layer F.Cu) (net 18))
 (segment (start 184.785 109.22) (end 184.785 104.775) (width 0.35) (layer F.Cu) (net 18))
 (segment (start 184.785 104.775) (end 185.42 104.14) (width 0.35) (layer B.Cu) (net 18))
 (segment (start 185.42 104.14) (end 185.42 100.33) (width 0.35) (layer B.Cu) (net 18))
 (segment (start 177.165 104.775) (end 180.34 104.775) (width 0.35) (layer B.Cu) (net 17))
 (segment (start 182.88 102.235) (end 182.88 100.33) (width 0.35) (layer B.Cu) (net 17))
 (segment (start 180.34 104.775) (end 182.88 102.235) (width 0.35) (layer B.Cu) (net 17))
 (segment (start 171.45 107.95) (end 172.085 107.95) (width 0.35) (layer F.Cu) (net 24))
 (segment (start 172.085 107.95) (end 173.355 109.22) (width 0.35) (layer F.Cu) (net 24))
 (segment (start 173.355 109.22) (end 177.165 109.22) (width 0.35) (layer F.Cu) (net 24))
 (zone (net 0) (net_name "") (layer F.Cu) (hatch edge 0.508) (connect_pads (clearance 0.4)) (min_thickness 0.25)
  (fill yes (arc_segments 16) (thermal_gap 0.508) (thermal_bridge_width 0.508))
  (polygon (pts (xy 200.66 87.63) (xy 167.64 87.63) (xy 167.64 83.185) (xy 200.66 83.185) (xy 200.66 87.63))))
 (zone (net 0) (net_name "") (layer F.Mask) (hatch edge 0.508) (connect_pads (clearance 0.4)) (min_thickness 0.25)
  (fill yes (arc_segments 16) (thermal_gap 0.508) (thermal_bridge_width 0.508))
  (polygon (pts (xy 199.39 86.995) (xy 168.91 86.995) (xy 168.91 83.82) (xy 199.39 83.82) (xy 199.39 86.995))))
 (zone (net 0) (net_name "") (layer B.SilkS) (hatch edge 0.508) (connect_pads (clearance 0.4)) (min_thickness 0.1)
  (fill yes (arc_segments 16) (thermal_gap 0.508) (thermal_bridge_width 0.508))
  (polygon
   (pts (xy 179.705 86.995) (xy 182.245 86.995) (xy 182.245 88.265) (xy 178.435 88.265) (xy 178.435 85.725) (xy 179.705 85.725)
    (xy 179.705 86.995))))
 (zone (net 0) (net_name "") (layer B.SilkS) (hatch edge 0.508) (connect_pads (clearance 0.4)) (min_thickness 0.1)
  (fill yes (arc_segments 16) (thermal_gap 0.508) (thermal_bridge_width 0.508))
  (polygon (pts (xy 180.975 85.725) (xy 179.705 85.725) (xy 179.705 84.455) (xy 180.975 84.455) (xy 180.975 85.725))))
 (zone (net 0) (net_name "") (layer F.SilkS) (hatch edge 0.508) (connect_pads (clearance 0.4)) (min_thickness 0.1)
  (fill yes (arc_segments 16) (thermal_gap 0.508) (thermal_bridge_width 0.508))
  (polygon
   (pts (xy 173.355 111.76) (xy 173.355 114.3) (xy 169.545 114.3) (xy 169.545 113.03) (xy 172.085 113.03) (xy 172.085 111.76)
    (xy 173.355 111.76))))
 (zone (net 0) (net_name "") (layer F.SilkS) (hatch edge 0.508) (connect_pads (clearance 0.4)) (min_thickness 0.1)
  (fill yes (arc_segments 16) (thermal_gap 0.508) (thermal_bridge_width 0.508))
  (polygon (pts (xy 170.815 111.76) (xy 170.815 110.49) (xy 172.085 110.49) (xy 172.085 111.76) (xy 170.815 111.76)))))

